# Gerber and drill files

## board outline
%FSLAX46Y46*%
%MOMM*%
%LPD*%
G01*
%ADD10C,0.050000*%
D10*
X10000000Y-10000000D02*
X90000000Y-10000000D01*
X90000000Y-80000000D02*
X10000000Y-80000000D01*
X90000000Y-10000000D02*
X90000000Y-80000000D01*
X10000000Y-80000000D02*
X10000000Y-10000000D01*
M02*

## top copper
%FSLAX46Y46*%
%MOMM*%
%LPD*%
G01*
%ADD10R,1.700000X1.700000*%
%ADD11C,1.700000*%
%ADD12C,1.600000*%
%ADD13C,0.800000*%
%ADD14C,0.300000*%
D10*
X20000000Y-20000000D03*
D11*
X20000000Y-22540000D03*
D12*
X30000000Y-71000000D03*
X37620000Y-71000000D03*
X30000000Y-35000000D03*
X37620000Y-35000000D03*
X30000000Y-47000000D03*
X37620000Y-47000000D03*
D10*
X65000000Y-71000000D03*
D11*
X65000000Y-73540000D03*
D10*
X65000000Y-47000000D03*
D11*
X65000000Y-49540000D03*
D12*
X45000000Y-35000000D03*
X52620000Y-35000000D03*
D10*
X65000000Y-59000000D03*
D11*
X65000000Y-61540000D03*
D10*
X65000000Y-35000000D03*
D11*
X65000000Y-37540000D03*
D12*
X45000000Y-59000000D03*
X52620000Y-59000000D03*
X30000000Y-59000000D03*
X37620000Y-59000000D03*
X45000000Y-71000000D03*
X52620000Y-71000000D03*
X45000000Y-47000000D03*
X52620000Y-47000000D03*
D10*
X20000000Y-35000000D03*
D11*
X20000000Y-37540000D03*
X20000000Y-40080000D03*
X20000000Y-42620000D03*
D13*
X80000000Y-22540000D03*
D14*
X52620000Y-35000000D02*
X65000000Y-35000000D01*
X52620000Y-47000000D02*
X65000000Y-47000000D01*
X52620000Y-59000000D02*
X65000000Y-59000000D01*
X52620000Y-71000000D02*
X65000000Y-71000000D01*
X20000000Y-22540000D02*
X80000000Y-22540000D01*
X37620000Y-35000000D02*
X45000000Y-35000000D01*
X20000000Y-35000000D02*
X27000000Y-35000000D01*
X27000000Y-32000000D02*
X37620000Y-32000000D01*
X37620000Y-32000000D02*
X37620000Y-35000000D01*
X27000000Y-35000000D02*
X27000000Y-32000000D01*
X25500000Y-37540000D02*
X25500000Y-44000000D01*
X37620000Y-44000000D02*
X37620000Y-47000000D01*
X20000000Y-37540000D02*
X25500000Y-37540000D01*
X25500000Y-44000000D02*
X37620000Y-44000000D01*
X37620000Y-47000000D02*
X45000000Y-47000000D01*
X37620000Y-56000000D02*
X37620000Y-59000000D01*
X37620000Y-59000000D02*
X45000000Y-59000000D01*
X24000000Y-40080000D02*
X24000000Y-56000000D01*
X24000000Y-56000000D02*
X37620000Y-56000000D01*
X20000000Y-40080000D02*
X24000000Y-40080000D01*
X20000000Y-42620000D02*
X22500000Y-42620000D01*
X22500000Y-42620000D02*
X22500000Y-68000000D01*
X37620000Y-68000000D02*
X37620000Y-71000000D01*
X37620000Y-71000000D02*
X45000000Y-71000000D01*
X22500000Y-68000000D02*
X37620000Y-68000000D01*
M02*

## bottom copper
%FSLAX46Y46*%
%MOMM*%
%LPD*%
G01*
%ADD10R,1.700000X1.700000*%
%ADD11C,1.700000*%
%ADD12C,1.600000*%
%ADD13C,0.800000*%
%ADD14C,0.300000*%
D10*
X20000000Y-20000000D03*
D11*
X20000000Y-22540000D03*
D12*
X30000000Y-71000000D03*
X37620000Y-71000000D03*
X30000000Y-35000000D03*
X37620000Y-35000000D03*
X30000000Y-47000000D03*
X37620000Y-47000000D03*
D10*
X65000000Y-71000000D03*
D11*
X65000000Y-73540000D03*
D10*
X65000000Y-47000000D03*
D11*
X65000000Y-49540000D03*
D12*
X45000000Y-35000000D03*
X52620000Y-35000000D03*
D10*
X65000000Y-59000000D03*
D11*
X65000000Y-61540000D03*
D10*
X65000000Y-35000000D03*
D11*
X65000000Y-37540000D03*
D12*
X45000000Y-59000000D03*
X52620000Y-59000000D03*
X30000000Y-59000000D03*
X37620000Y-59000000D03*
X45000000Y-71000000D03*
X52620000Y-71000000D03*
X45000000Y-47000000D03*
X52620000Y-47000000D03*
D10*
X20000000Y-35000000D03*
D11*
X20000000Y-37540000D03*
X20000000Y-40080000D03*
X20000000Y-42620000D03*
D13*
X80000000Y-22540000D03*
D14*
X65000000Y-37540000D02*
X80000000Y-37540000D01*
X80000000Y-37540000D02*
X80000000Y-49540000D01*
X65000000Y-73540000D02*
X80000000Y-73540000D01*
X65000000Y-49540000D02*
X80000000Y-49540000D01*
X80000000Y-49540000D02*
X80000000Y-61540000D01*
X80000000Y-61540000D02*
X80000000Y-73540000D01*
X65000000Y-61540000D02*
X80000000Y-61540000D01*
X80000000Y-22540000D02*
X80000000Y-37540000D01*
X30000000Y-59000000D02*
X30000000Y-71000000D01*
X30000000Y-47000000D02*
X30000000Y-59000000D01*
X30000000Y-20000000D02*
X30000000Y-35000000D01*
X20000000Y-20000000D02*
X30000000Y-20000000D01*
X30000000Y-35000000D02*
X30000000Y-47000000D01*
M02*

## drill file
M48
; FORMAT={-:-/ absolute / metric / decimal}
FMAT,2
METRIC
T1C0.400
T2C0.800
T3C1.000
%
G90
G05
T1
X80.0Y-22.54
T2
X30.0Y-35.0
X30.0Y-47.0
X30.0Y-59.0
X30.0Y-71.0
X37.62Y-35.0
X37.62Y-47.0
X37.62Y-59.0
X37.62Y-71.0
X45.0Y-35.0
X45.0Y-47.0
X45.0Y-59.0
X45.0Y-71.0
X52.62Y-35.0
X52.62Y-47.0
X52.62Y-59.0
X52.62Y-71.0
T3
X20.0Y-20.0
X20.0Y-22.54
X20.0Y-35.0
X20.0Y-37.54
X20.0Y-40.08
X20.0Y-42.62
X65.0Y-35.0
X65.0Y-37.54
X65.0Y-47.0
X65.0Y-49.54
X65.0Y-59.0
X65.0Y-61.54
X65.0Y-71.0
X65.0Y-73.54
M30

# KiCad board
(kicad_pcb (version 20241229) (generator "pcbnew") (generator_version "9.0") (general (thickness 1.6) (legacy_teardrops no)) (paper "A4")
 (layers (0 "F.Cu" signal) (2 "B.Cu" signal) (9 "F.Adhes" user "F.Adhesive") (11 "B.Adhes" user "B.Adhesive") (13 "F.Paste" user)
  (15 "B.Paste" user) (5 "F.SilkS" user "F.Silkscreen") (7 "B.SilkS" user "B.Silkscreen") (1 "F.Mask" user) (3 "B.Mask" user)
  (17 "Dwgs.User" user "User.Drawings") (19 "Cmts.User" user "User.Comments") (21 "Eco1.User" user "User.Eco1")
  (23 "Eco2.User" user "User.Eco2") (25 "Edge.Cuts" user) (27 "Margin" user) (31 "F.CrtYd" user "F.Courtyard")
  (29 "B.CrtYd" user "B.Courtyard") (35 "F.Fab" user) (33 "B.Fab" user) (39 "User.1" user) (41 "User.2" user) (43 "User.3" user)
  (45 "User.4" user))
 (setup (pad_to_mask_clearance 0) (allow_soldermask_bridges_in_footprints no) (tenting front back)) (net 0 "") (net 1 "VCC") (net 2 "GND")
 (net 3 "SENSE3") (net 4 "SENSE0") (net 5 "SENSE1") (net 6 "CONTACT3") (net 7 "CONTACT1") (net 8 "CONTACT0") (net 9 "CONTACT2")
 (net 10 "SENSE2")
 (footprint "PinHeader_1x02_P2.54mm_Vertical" (layer "F.Cu") (at 20 20)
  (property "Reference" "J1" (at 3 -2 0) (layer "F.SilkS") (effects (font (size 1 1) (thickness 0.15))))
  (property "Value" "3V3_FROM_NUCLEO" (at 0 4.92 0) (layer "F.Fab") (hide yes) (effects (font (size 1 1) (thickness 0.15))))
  (pad "1" thru_hole rect (at 0 0) (size 1.7 1.7) (drill 1) (layers "*.Cu" "*.Mask") (remove_unused_layers no) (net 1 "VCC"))
  (pad "2" thru_hole circle (at 0 2.54) (size 1.7 1.7) (drill 1) (layers "*.Cu" "*.Mask") (remove_unused_layers no) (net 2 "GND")))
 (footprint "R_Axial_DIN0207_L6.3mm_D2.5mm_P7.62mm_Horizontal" (layer "F.Cu") (at 30 71)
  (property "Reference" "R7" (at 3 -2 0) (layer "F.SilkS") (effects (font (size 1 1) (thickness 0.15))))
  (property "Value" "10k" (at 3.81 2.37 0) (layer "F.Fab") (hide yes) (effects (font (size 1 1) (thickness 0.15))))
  (pad "1" thru_hole circle (at 0 0) (size 1.6 1.6) (drill 0.8) (layers "*.Cu" "*.Mask") (remove_unused_layers no) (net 1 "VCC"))
  (pad "2" thru_hole circle (at 7.62 0) (size 1.6 1.6) (drill 0.8) (layers "*.Cu" "*.Mask") (remove_unused_layers no) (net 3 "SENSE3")))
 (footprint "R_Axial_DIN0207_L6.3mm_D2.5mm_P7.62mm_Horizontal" (layer "F.Cu") (at 30 35)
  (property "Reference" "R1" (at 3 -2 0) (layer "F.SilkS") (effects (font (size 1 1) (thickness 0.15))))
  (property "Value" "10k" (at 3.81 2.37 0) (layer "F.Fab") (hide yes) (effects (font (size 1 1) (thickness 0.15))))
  (pad "1" thru_hole circle (at 0 0) (size 1.6 1.6) (drill 0.8) (layers "*.Cu" "*.Mask") (remove_unused_layers no) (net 1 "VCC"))
  (pad "2" thru_hole circle (at 7.62 0) (size 1.6 1.6) (drill 0.8) (layers "*.Cu" "*.Mask") (remove_unused_layers no) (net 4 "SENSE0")))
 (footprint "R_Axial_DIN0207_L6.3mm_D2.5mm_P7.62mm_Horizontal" (layer "F.Cu") (at 30 47)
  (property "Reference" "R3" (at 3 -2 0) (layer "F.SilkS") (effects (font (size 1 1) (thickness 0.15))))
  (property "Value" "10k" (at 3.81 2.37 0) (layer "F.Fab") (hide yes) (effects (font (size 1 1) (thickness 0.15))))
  (pad "1" thru_hole circle (at 0 0) (size 1.6 1.6) (drill 0.8) (layers "*.Cu" "*.Mask") (remove_unused_layers no) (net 1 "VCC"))
  (pad "2" thru_hole circle (at 7.62 0) (size 1.6 1.6) (drill 0.8) (layers "*.Cu" "*.Mask") (remove_unused_layers no) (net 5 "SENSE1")))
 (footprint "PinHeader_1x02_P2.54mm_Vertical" (layer "F.Cu") (at 65 71)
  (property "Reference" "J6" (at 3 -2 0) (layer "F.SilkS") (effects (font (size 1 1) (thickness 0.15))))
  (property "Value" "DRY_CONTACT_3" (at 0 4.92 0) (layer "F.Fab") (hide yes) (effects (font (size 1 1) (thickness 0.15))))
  (pad "1" thru_hole rect (at 0 0) (size 1.7 1.7) (drill 1) (layers "*.Cu" "*.Mask") (remove_unused_layers no) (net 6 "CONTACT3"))
  (pad "2" thru_hole circle (at 0 2.54) (size 1.7 1.7) (drill 1) (layers "*.Cu" "*.Mask") (remove_unused_layers no) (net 2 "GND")))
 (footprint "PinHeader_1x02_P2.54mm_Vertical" (layer "F.Cu") (at 65 47)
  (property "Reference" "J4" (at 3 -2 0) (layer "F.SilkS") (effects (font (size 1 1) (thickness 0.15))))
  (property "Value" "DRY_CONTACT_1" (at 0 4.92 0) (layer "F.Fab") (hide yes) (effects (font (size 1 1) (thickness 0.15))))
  (pad "1" thru_hole rect (at 0 0) (size 1.7 1.7) (drill 1) (layers "*.Cu" "*.Mask") (remove_unused_layers no) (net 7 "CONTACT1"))
  (pad "2" thru_hole circle (at 0 2.54) (size 1.7 1.7) (drill 1) (layers "*.Cu" "*.Mask") (remove_unused_layers no) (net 2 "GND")))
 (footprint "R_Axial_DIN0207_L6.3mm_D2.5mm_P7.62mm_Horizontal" (layer "F.Cu") (at 45 35)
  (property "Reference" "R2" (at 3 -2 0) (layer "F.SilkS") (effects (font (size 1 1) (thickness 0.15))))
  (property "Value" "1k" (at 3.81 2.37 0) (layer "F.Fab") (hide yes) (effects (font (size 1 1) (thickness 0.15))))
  (pad "1" thru_hole circle (at 0 0) (size 1.6 1.6) (drill 0.8) (layers "*.Cu" "*.Mask") (remove_unused_layers no) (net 4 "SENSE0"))
  (pad "2" thru_hole circle (at 7.62 0) (size 1.6 1.6) (drill 0.8) (layers "*.Cu" "*.Mask") (remove_unused_layers no) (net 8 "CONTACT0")))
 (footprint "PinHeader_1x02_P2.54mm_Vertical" (layer "F.Cu") (at 65 59)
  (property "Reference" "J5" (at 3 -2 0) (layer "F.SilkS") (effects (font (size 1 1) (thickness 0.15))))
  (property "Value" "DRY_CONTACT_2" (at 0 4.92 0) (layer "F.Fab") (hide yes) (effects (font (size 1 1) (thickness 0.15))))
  (pad "1" thru_hole rect (at 0 0) (size 1.7 1.7) (drill 1) (layers "*.Cu" "*.Mask") (remove_unused_layers no) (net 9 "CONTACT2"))
  (pad "2" thru_hole circle (at 0 2.54) (size 1.7 1.7) (drill 1) (layers "*.Cu" "*.Mask") (remove_unused_layers no) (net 2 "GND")))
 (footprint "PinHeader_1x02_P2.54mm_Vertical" (layer "F.Cu") (at 65 35)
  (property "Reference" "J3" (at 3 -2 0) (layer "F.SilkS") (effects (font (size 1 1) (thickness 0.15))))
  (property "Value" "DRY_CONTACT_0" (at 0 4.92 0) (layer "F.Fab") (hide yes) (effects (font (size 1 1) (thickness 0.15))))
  (pad "1" thru_hole rect (at 0 0) (size 1.7 1.7) (drill 1) (layers "*.Cu" "*.Mask") (remove_unused_layers no) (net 8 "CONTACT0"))
  (pad "2" thru_hole circle (at 0 2.54) (size 1.7 1.7) (drill 1) (layers "*.Cu" "*.Mask") (remove_unused_layers no) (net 2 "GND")))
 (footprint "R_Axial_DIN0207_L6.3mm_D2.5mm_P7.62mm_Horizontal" (layer "F.Cu") (at 45 59)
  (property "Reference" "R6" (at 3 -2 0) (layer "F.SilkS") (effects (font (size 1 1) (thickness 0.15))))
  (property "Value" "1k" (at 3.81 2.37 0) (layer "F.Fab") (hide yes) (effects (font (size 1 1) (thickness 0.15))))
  (pad "1" thru_hole circle (at 0 0) (size 1.6 1.6) (drill 0.8) (layers "*.Cu" "*.Mask") (remove_unused_layers no) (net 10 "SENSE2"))
  (pad "2" thru_hole circle (at 7.62 0) (size 1.6 1.6) (drill 0.8) (layers "*.Cu" "*.Mask") (remove_unused_layers no) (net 9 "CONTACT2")))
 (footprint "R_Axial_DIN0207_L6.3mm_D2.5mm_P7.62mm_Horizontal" (layer "F.Cu") (at 30 59)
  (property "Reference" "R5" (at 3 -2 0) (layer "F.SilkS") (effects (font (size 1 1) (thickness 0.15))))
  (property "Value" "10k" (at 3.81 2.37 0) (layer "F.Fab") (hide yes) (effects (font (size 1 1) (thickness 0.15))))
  (pad "1" thru_hole circle (at 0 0) (size 1.6 1.6) (drill 0.8) (layers "*.Cu" "*.Mask") (remove_unused_layers no) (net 1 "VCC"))
  (pad "2" thru_hole circle (at 7.62 0) (size 1.6 1.6) (drill 0.8) (layers "*.Cu" "*.Mask") (remove_unused_layers no) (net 10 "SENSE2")))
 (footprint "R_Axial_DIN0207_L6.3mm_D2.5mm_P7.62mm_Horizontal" (layer "F.Cu") (at 45 71)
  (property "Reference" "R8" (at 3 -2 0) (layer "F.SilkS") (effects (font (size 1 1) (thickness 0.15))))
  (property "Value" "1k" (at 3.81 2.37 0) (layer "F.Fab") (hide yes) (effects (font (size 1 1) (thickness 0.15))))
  (pad "1" thru_hole circle (at 0 0) (size 1.6 1.6) (drill 0.8) (layers "*.Cu" "*.Mask") (remove_unused_layers no) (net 3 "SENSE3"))
  (pad "2" thru_hole circle (at 7.62 0) (size 1.6 1.6) (drill 0.8) (layers "*.Cu" "*.Mask") (remove_unused_layers no) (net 6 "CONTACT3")))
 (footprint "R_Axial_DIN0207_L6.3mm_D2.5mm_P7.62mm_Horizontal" (layer "F.Cu") (at 45 47)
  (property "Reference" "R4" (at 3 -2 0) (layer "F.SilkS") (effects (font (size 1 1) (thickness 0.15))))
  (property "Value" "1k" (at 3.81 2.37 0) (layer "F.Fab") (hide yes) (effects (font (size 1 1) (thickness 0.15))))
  (pad "1" thru_hole circle (at 0 0) (size 1.6 1.6) (drill 0.8) (layers "*.Cu" "*.Mask") (remove_unused_layers no) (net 5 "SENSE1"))
  (pad "2" thru_hole circle (at 7.62 0) (size 1.6 1.6) (drill 0.8) (layers "*.Cu" "*.Mask") (remove_unused_layers no) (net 7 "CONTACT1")))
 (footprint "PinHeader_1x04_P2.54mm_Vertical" (layer "F.Cu") (at 20 35)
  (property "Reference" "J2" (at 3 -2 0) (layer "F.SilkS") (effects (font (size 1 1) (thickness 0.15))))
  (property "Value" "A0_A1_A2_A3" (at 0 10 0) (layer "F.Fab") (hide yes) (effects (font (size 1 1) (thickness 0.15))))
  (pad "1" thru_hole rect (at 0 0) (size 1.7 1.7) (drill 1) (layers "*.Cu" "*.Mask") (remove_unused_layers no) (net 4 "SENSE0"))
  (pad "2" thru_hole circle (at 0 2.54) (size 1.7 1.7) (drill 1) (layers "*.Cu" "*.Mask") (remove_unused_layers no) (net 5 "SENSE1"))
  (pad "3" thru_hole circle (at 0 5.08) (size 1.7 1.7) (drill 1) (layers "*.Cu" "*.Mask") (remove_unused_layers no) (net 10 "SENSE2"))
  (pad "4" thru_hole circle (at 0 7.62) (size 1.7 1.7) (drill 1) (layers "*.Cu" "*.Mask") (remove_unused_layers no) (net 3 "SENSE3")))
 (gr_line (start 10 10) (end 90 10) (stroke (width 0.05) (type default)) (layer "Edge.Cuts"))
 (gr_line (start 90 80) (end 10 80) (stroke (width 0.05) (type default)) (layer "Edge.Cuts"))
 (gr_line (start 90 10) (end 90 80) (stroke (width 0.05) (type default)) (layer "Edge.Cuts"))
 (gr_line (start 10 80) (end 10 10) (stroke (width 0.05) (type default)) (layer "Edge.Cuts"))
 (segment (start 52.62 35) (end 65 35) (width 0.3) (layer "F.Cu") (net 8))
 (segment (start 52.62 47) (end 65 47) (width 0.3) (layer "F.Cu") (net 7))
 (segment (start 52.62 59) (end 65 59) (width 0.3) (layer "F.Cu") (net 9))
 (segment (start 52.62 71) (end 65 71) (width 0.3) (layer "F.Cu") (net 6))
 (segment (start 20 22.54) (end 80 22.54) (width 0.3) (layer "F.Cu") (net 2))
 (via (at 80 22.54) (size 0.8) (drill 0.4) (layers "F.Cu" "B.Cu") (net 2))
 (segment (start 65 37.54) (end 80 37.54) (width 0.3) (layer "B.Cu") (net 2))
 (segment (start 80 37.54) (end 80 49.54) (width 0.3) (layer "B.Cu") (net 2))
 (segment (start 65 73.54) (end 80 73.54) (width 0.3) (layer "B.Cu") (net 2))
 (segment (start 65 49.54) (end 80 49.54) (width 0.3) (layer "B.Cu") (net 2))
 (segment (start 80 49.54) (end 80 61.54) (width 0.3) (layer "B.Cu") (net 2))
 (segment (start 80 61.54) (end 80 73.54) (width 0.3) (layer "B.Cu") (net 2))
 (segment (start 65 61.54) (end 80 61.54) (width 0.3) (layer "B.Cu") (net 2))
 (segment (start 80 22.54) (end 80 37.54) (width 0.3) (layer "B.Cu") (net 2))
 (segment (start 37.62 35) (end 45 35) (width 0.3) (layer "F.Cu") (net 4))
 (segment (start 20 35) (end 27 35) (width 0.3) (layer "F.Cu") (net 4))
 (segment (start 27 32) (end 37.62 32) (width 0.3) (layer "F.Cu") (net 4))
 (segment (start 37.62 32) (end 37.62 35) (width 0.3) (layer "F.Cu") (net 4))
 (segment (start 27 35) (end 27 32) (width 0.3) (layer "F.Cu") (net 4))
 (segment (start 25.5 37.54) (end 25.5 44) (width 0.3) (layer "F.Cu") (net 5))
 (segment (start 37.62 44) (end 37.62 47) (width 0.3) (layer "F.Cu") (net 5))
 (segment (start 20 37.54) (end 25.5 37.54) (width 0.3) (layer "F.Cu") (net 5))
 (segment (start 25.5 44) (end 37.62 44) (width 0.3) (layer "F.Cu") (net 5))
 (segment (start 37.62 47) (end 45 47) (width 0.3) (layer "F.Cu") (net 5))
 (segment (start 37.62 56) (end 37.62 59) (width 0.3) (layer "F.Cu") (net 10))
 (segment (start 37.62 59) (end 45 59) (width 0.3) (layer "F.Cu") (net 10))
 (segment (start 24 40.08) (end 24 56) (width 0.3) (layer "F.Cu") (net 10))
 (segment (start 24 56) (end 37.62 56) (width 0.3) (layer "F.Cu") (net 10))
 (segment (start 20 40.08) (end 24 40.08) (width 0.3) (layer "F.Cu") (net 10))
 (segment (start 20 42.62) (end 22.5 42.62) (width 0.3) (layer "F.Cu") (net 3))
 (segment (start 22.5 42.62) (end 22.5 68) (width 0.3) (layer "F.Cu") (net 3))
 (segment (start 37.62 68) (end 37.62 71) (width 0.3) (layer "F.Cu") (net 3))
 (segment (start 37.62 71) (end 45 71) (width 0.3) (layer "F.Cu") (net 3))
 (segment (start 22.5 68) (end 37.62 68) (width 0.3) (layer "F.Cu") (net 3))
 (segment (start 30 59) (end 30 71) (width 0.3) (layer "B.Cu") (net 1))
 (segment (start 30 47) (end 30 59) (width 0.3) (layer "B.Cu") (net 1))
 (segment (start 30 20) (end 30 35) (width 0.3) (layer "B.Cu") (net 1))
 (segment (start 20 20) (end 30 20) (width 0.3) (layer "B.Cu") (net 1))
 (segment (start 30 35) (end 30 47) (width 0.3) (layer "B.Cu") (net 1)))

